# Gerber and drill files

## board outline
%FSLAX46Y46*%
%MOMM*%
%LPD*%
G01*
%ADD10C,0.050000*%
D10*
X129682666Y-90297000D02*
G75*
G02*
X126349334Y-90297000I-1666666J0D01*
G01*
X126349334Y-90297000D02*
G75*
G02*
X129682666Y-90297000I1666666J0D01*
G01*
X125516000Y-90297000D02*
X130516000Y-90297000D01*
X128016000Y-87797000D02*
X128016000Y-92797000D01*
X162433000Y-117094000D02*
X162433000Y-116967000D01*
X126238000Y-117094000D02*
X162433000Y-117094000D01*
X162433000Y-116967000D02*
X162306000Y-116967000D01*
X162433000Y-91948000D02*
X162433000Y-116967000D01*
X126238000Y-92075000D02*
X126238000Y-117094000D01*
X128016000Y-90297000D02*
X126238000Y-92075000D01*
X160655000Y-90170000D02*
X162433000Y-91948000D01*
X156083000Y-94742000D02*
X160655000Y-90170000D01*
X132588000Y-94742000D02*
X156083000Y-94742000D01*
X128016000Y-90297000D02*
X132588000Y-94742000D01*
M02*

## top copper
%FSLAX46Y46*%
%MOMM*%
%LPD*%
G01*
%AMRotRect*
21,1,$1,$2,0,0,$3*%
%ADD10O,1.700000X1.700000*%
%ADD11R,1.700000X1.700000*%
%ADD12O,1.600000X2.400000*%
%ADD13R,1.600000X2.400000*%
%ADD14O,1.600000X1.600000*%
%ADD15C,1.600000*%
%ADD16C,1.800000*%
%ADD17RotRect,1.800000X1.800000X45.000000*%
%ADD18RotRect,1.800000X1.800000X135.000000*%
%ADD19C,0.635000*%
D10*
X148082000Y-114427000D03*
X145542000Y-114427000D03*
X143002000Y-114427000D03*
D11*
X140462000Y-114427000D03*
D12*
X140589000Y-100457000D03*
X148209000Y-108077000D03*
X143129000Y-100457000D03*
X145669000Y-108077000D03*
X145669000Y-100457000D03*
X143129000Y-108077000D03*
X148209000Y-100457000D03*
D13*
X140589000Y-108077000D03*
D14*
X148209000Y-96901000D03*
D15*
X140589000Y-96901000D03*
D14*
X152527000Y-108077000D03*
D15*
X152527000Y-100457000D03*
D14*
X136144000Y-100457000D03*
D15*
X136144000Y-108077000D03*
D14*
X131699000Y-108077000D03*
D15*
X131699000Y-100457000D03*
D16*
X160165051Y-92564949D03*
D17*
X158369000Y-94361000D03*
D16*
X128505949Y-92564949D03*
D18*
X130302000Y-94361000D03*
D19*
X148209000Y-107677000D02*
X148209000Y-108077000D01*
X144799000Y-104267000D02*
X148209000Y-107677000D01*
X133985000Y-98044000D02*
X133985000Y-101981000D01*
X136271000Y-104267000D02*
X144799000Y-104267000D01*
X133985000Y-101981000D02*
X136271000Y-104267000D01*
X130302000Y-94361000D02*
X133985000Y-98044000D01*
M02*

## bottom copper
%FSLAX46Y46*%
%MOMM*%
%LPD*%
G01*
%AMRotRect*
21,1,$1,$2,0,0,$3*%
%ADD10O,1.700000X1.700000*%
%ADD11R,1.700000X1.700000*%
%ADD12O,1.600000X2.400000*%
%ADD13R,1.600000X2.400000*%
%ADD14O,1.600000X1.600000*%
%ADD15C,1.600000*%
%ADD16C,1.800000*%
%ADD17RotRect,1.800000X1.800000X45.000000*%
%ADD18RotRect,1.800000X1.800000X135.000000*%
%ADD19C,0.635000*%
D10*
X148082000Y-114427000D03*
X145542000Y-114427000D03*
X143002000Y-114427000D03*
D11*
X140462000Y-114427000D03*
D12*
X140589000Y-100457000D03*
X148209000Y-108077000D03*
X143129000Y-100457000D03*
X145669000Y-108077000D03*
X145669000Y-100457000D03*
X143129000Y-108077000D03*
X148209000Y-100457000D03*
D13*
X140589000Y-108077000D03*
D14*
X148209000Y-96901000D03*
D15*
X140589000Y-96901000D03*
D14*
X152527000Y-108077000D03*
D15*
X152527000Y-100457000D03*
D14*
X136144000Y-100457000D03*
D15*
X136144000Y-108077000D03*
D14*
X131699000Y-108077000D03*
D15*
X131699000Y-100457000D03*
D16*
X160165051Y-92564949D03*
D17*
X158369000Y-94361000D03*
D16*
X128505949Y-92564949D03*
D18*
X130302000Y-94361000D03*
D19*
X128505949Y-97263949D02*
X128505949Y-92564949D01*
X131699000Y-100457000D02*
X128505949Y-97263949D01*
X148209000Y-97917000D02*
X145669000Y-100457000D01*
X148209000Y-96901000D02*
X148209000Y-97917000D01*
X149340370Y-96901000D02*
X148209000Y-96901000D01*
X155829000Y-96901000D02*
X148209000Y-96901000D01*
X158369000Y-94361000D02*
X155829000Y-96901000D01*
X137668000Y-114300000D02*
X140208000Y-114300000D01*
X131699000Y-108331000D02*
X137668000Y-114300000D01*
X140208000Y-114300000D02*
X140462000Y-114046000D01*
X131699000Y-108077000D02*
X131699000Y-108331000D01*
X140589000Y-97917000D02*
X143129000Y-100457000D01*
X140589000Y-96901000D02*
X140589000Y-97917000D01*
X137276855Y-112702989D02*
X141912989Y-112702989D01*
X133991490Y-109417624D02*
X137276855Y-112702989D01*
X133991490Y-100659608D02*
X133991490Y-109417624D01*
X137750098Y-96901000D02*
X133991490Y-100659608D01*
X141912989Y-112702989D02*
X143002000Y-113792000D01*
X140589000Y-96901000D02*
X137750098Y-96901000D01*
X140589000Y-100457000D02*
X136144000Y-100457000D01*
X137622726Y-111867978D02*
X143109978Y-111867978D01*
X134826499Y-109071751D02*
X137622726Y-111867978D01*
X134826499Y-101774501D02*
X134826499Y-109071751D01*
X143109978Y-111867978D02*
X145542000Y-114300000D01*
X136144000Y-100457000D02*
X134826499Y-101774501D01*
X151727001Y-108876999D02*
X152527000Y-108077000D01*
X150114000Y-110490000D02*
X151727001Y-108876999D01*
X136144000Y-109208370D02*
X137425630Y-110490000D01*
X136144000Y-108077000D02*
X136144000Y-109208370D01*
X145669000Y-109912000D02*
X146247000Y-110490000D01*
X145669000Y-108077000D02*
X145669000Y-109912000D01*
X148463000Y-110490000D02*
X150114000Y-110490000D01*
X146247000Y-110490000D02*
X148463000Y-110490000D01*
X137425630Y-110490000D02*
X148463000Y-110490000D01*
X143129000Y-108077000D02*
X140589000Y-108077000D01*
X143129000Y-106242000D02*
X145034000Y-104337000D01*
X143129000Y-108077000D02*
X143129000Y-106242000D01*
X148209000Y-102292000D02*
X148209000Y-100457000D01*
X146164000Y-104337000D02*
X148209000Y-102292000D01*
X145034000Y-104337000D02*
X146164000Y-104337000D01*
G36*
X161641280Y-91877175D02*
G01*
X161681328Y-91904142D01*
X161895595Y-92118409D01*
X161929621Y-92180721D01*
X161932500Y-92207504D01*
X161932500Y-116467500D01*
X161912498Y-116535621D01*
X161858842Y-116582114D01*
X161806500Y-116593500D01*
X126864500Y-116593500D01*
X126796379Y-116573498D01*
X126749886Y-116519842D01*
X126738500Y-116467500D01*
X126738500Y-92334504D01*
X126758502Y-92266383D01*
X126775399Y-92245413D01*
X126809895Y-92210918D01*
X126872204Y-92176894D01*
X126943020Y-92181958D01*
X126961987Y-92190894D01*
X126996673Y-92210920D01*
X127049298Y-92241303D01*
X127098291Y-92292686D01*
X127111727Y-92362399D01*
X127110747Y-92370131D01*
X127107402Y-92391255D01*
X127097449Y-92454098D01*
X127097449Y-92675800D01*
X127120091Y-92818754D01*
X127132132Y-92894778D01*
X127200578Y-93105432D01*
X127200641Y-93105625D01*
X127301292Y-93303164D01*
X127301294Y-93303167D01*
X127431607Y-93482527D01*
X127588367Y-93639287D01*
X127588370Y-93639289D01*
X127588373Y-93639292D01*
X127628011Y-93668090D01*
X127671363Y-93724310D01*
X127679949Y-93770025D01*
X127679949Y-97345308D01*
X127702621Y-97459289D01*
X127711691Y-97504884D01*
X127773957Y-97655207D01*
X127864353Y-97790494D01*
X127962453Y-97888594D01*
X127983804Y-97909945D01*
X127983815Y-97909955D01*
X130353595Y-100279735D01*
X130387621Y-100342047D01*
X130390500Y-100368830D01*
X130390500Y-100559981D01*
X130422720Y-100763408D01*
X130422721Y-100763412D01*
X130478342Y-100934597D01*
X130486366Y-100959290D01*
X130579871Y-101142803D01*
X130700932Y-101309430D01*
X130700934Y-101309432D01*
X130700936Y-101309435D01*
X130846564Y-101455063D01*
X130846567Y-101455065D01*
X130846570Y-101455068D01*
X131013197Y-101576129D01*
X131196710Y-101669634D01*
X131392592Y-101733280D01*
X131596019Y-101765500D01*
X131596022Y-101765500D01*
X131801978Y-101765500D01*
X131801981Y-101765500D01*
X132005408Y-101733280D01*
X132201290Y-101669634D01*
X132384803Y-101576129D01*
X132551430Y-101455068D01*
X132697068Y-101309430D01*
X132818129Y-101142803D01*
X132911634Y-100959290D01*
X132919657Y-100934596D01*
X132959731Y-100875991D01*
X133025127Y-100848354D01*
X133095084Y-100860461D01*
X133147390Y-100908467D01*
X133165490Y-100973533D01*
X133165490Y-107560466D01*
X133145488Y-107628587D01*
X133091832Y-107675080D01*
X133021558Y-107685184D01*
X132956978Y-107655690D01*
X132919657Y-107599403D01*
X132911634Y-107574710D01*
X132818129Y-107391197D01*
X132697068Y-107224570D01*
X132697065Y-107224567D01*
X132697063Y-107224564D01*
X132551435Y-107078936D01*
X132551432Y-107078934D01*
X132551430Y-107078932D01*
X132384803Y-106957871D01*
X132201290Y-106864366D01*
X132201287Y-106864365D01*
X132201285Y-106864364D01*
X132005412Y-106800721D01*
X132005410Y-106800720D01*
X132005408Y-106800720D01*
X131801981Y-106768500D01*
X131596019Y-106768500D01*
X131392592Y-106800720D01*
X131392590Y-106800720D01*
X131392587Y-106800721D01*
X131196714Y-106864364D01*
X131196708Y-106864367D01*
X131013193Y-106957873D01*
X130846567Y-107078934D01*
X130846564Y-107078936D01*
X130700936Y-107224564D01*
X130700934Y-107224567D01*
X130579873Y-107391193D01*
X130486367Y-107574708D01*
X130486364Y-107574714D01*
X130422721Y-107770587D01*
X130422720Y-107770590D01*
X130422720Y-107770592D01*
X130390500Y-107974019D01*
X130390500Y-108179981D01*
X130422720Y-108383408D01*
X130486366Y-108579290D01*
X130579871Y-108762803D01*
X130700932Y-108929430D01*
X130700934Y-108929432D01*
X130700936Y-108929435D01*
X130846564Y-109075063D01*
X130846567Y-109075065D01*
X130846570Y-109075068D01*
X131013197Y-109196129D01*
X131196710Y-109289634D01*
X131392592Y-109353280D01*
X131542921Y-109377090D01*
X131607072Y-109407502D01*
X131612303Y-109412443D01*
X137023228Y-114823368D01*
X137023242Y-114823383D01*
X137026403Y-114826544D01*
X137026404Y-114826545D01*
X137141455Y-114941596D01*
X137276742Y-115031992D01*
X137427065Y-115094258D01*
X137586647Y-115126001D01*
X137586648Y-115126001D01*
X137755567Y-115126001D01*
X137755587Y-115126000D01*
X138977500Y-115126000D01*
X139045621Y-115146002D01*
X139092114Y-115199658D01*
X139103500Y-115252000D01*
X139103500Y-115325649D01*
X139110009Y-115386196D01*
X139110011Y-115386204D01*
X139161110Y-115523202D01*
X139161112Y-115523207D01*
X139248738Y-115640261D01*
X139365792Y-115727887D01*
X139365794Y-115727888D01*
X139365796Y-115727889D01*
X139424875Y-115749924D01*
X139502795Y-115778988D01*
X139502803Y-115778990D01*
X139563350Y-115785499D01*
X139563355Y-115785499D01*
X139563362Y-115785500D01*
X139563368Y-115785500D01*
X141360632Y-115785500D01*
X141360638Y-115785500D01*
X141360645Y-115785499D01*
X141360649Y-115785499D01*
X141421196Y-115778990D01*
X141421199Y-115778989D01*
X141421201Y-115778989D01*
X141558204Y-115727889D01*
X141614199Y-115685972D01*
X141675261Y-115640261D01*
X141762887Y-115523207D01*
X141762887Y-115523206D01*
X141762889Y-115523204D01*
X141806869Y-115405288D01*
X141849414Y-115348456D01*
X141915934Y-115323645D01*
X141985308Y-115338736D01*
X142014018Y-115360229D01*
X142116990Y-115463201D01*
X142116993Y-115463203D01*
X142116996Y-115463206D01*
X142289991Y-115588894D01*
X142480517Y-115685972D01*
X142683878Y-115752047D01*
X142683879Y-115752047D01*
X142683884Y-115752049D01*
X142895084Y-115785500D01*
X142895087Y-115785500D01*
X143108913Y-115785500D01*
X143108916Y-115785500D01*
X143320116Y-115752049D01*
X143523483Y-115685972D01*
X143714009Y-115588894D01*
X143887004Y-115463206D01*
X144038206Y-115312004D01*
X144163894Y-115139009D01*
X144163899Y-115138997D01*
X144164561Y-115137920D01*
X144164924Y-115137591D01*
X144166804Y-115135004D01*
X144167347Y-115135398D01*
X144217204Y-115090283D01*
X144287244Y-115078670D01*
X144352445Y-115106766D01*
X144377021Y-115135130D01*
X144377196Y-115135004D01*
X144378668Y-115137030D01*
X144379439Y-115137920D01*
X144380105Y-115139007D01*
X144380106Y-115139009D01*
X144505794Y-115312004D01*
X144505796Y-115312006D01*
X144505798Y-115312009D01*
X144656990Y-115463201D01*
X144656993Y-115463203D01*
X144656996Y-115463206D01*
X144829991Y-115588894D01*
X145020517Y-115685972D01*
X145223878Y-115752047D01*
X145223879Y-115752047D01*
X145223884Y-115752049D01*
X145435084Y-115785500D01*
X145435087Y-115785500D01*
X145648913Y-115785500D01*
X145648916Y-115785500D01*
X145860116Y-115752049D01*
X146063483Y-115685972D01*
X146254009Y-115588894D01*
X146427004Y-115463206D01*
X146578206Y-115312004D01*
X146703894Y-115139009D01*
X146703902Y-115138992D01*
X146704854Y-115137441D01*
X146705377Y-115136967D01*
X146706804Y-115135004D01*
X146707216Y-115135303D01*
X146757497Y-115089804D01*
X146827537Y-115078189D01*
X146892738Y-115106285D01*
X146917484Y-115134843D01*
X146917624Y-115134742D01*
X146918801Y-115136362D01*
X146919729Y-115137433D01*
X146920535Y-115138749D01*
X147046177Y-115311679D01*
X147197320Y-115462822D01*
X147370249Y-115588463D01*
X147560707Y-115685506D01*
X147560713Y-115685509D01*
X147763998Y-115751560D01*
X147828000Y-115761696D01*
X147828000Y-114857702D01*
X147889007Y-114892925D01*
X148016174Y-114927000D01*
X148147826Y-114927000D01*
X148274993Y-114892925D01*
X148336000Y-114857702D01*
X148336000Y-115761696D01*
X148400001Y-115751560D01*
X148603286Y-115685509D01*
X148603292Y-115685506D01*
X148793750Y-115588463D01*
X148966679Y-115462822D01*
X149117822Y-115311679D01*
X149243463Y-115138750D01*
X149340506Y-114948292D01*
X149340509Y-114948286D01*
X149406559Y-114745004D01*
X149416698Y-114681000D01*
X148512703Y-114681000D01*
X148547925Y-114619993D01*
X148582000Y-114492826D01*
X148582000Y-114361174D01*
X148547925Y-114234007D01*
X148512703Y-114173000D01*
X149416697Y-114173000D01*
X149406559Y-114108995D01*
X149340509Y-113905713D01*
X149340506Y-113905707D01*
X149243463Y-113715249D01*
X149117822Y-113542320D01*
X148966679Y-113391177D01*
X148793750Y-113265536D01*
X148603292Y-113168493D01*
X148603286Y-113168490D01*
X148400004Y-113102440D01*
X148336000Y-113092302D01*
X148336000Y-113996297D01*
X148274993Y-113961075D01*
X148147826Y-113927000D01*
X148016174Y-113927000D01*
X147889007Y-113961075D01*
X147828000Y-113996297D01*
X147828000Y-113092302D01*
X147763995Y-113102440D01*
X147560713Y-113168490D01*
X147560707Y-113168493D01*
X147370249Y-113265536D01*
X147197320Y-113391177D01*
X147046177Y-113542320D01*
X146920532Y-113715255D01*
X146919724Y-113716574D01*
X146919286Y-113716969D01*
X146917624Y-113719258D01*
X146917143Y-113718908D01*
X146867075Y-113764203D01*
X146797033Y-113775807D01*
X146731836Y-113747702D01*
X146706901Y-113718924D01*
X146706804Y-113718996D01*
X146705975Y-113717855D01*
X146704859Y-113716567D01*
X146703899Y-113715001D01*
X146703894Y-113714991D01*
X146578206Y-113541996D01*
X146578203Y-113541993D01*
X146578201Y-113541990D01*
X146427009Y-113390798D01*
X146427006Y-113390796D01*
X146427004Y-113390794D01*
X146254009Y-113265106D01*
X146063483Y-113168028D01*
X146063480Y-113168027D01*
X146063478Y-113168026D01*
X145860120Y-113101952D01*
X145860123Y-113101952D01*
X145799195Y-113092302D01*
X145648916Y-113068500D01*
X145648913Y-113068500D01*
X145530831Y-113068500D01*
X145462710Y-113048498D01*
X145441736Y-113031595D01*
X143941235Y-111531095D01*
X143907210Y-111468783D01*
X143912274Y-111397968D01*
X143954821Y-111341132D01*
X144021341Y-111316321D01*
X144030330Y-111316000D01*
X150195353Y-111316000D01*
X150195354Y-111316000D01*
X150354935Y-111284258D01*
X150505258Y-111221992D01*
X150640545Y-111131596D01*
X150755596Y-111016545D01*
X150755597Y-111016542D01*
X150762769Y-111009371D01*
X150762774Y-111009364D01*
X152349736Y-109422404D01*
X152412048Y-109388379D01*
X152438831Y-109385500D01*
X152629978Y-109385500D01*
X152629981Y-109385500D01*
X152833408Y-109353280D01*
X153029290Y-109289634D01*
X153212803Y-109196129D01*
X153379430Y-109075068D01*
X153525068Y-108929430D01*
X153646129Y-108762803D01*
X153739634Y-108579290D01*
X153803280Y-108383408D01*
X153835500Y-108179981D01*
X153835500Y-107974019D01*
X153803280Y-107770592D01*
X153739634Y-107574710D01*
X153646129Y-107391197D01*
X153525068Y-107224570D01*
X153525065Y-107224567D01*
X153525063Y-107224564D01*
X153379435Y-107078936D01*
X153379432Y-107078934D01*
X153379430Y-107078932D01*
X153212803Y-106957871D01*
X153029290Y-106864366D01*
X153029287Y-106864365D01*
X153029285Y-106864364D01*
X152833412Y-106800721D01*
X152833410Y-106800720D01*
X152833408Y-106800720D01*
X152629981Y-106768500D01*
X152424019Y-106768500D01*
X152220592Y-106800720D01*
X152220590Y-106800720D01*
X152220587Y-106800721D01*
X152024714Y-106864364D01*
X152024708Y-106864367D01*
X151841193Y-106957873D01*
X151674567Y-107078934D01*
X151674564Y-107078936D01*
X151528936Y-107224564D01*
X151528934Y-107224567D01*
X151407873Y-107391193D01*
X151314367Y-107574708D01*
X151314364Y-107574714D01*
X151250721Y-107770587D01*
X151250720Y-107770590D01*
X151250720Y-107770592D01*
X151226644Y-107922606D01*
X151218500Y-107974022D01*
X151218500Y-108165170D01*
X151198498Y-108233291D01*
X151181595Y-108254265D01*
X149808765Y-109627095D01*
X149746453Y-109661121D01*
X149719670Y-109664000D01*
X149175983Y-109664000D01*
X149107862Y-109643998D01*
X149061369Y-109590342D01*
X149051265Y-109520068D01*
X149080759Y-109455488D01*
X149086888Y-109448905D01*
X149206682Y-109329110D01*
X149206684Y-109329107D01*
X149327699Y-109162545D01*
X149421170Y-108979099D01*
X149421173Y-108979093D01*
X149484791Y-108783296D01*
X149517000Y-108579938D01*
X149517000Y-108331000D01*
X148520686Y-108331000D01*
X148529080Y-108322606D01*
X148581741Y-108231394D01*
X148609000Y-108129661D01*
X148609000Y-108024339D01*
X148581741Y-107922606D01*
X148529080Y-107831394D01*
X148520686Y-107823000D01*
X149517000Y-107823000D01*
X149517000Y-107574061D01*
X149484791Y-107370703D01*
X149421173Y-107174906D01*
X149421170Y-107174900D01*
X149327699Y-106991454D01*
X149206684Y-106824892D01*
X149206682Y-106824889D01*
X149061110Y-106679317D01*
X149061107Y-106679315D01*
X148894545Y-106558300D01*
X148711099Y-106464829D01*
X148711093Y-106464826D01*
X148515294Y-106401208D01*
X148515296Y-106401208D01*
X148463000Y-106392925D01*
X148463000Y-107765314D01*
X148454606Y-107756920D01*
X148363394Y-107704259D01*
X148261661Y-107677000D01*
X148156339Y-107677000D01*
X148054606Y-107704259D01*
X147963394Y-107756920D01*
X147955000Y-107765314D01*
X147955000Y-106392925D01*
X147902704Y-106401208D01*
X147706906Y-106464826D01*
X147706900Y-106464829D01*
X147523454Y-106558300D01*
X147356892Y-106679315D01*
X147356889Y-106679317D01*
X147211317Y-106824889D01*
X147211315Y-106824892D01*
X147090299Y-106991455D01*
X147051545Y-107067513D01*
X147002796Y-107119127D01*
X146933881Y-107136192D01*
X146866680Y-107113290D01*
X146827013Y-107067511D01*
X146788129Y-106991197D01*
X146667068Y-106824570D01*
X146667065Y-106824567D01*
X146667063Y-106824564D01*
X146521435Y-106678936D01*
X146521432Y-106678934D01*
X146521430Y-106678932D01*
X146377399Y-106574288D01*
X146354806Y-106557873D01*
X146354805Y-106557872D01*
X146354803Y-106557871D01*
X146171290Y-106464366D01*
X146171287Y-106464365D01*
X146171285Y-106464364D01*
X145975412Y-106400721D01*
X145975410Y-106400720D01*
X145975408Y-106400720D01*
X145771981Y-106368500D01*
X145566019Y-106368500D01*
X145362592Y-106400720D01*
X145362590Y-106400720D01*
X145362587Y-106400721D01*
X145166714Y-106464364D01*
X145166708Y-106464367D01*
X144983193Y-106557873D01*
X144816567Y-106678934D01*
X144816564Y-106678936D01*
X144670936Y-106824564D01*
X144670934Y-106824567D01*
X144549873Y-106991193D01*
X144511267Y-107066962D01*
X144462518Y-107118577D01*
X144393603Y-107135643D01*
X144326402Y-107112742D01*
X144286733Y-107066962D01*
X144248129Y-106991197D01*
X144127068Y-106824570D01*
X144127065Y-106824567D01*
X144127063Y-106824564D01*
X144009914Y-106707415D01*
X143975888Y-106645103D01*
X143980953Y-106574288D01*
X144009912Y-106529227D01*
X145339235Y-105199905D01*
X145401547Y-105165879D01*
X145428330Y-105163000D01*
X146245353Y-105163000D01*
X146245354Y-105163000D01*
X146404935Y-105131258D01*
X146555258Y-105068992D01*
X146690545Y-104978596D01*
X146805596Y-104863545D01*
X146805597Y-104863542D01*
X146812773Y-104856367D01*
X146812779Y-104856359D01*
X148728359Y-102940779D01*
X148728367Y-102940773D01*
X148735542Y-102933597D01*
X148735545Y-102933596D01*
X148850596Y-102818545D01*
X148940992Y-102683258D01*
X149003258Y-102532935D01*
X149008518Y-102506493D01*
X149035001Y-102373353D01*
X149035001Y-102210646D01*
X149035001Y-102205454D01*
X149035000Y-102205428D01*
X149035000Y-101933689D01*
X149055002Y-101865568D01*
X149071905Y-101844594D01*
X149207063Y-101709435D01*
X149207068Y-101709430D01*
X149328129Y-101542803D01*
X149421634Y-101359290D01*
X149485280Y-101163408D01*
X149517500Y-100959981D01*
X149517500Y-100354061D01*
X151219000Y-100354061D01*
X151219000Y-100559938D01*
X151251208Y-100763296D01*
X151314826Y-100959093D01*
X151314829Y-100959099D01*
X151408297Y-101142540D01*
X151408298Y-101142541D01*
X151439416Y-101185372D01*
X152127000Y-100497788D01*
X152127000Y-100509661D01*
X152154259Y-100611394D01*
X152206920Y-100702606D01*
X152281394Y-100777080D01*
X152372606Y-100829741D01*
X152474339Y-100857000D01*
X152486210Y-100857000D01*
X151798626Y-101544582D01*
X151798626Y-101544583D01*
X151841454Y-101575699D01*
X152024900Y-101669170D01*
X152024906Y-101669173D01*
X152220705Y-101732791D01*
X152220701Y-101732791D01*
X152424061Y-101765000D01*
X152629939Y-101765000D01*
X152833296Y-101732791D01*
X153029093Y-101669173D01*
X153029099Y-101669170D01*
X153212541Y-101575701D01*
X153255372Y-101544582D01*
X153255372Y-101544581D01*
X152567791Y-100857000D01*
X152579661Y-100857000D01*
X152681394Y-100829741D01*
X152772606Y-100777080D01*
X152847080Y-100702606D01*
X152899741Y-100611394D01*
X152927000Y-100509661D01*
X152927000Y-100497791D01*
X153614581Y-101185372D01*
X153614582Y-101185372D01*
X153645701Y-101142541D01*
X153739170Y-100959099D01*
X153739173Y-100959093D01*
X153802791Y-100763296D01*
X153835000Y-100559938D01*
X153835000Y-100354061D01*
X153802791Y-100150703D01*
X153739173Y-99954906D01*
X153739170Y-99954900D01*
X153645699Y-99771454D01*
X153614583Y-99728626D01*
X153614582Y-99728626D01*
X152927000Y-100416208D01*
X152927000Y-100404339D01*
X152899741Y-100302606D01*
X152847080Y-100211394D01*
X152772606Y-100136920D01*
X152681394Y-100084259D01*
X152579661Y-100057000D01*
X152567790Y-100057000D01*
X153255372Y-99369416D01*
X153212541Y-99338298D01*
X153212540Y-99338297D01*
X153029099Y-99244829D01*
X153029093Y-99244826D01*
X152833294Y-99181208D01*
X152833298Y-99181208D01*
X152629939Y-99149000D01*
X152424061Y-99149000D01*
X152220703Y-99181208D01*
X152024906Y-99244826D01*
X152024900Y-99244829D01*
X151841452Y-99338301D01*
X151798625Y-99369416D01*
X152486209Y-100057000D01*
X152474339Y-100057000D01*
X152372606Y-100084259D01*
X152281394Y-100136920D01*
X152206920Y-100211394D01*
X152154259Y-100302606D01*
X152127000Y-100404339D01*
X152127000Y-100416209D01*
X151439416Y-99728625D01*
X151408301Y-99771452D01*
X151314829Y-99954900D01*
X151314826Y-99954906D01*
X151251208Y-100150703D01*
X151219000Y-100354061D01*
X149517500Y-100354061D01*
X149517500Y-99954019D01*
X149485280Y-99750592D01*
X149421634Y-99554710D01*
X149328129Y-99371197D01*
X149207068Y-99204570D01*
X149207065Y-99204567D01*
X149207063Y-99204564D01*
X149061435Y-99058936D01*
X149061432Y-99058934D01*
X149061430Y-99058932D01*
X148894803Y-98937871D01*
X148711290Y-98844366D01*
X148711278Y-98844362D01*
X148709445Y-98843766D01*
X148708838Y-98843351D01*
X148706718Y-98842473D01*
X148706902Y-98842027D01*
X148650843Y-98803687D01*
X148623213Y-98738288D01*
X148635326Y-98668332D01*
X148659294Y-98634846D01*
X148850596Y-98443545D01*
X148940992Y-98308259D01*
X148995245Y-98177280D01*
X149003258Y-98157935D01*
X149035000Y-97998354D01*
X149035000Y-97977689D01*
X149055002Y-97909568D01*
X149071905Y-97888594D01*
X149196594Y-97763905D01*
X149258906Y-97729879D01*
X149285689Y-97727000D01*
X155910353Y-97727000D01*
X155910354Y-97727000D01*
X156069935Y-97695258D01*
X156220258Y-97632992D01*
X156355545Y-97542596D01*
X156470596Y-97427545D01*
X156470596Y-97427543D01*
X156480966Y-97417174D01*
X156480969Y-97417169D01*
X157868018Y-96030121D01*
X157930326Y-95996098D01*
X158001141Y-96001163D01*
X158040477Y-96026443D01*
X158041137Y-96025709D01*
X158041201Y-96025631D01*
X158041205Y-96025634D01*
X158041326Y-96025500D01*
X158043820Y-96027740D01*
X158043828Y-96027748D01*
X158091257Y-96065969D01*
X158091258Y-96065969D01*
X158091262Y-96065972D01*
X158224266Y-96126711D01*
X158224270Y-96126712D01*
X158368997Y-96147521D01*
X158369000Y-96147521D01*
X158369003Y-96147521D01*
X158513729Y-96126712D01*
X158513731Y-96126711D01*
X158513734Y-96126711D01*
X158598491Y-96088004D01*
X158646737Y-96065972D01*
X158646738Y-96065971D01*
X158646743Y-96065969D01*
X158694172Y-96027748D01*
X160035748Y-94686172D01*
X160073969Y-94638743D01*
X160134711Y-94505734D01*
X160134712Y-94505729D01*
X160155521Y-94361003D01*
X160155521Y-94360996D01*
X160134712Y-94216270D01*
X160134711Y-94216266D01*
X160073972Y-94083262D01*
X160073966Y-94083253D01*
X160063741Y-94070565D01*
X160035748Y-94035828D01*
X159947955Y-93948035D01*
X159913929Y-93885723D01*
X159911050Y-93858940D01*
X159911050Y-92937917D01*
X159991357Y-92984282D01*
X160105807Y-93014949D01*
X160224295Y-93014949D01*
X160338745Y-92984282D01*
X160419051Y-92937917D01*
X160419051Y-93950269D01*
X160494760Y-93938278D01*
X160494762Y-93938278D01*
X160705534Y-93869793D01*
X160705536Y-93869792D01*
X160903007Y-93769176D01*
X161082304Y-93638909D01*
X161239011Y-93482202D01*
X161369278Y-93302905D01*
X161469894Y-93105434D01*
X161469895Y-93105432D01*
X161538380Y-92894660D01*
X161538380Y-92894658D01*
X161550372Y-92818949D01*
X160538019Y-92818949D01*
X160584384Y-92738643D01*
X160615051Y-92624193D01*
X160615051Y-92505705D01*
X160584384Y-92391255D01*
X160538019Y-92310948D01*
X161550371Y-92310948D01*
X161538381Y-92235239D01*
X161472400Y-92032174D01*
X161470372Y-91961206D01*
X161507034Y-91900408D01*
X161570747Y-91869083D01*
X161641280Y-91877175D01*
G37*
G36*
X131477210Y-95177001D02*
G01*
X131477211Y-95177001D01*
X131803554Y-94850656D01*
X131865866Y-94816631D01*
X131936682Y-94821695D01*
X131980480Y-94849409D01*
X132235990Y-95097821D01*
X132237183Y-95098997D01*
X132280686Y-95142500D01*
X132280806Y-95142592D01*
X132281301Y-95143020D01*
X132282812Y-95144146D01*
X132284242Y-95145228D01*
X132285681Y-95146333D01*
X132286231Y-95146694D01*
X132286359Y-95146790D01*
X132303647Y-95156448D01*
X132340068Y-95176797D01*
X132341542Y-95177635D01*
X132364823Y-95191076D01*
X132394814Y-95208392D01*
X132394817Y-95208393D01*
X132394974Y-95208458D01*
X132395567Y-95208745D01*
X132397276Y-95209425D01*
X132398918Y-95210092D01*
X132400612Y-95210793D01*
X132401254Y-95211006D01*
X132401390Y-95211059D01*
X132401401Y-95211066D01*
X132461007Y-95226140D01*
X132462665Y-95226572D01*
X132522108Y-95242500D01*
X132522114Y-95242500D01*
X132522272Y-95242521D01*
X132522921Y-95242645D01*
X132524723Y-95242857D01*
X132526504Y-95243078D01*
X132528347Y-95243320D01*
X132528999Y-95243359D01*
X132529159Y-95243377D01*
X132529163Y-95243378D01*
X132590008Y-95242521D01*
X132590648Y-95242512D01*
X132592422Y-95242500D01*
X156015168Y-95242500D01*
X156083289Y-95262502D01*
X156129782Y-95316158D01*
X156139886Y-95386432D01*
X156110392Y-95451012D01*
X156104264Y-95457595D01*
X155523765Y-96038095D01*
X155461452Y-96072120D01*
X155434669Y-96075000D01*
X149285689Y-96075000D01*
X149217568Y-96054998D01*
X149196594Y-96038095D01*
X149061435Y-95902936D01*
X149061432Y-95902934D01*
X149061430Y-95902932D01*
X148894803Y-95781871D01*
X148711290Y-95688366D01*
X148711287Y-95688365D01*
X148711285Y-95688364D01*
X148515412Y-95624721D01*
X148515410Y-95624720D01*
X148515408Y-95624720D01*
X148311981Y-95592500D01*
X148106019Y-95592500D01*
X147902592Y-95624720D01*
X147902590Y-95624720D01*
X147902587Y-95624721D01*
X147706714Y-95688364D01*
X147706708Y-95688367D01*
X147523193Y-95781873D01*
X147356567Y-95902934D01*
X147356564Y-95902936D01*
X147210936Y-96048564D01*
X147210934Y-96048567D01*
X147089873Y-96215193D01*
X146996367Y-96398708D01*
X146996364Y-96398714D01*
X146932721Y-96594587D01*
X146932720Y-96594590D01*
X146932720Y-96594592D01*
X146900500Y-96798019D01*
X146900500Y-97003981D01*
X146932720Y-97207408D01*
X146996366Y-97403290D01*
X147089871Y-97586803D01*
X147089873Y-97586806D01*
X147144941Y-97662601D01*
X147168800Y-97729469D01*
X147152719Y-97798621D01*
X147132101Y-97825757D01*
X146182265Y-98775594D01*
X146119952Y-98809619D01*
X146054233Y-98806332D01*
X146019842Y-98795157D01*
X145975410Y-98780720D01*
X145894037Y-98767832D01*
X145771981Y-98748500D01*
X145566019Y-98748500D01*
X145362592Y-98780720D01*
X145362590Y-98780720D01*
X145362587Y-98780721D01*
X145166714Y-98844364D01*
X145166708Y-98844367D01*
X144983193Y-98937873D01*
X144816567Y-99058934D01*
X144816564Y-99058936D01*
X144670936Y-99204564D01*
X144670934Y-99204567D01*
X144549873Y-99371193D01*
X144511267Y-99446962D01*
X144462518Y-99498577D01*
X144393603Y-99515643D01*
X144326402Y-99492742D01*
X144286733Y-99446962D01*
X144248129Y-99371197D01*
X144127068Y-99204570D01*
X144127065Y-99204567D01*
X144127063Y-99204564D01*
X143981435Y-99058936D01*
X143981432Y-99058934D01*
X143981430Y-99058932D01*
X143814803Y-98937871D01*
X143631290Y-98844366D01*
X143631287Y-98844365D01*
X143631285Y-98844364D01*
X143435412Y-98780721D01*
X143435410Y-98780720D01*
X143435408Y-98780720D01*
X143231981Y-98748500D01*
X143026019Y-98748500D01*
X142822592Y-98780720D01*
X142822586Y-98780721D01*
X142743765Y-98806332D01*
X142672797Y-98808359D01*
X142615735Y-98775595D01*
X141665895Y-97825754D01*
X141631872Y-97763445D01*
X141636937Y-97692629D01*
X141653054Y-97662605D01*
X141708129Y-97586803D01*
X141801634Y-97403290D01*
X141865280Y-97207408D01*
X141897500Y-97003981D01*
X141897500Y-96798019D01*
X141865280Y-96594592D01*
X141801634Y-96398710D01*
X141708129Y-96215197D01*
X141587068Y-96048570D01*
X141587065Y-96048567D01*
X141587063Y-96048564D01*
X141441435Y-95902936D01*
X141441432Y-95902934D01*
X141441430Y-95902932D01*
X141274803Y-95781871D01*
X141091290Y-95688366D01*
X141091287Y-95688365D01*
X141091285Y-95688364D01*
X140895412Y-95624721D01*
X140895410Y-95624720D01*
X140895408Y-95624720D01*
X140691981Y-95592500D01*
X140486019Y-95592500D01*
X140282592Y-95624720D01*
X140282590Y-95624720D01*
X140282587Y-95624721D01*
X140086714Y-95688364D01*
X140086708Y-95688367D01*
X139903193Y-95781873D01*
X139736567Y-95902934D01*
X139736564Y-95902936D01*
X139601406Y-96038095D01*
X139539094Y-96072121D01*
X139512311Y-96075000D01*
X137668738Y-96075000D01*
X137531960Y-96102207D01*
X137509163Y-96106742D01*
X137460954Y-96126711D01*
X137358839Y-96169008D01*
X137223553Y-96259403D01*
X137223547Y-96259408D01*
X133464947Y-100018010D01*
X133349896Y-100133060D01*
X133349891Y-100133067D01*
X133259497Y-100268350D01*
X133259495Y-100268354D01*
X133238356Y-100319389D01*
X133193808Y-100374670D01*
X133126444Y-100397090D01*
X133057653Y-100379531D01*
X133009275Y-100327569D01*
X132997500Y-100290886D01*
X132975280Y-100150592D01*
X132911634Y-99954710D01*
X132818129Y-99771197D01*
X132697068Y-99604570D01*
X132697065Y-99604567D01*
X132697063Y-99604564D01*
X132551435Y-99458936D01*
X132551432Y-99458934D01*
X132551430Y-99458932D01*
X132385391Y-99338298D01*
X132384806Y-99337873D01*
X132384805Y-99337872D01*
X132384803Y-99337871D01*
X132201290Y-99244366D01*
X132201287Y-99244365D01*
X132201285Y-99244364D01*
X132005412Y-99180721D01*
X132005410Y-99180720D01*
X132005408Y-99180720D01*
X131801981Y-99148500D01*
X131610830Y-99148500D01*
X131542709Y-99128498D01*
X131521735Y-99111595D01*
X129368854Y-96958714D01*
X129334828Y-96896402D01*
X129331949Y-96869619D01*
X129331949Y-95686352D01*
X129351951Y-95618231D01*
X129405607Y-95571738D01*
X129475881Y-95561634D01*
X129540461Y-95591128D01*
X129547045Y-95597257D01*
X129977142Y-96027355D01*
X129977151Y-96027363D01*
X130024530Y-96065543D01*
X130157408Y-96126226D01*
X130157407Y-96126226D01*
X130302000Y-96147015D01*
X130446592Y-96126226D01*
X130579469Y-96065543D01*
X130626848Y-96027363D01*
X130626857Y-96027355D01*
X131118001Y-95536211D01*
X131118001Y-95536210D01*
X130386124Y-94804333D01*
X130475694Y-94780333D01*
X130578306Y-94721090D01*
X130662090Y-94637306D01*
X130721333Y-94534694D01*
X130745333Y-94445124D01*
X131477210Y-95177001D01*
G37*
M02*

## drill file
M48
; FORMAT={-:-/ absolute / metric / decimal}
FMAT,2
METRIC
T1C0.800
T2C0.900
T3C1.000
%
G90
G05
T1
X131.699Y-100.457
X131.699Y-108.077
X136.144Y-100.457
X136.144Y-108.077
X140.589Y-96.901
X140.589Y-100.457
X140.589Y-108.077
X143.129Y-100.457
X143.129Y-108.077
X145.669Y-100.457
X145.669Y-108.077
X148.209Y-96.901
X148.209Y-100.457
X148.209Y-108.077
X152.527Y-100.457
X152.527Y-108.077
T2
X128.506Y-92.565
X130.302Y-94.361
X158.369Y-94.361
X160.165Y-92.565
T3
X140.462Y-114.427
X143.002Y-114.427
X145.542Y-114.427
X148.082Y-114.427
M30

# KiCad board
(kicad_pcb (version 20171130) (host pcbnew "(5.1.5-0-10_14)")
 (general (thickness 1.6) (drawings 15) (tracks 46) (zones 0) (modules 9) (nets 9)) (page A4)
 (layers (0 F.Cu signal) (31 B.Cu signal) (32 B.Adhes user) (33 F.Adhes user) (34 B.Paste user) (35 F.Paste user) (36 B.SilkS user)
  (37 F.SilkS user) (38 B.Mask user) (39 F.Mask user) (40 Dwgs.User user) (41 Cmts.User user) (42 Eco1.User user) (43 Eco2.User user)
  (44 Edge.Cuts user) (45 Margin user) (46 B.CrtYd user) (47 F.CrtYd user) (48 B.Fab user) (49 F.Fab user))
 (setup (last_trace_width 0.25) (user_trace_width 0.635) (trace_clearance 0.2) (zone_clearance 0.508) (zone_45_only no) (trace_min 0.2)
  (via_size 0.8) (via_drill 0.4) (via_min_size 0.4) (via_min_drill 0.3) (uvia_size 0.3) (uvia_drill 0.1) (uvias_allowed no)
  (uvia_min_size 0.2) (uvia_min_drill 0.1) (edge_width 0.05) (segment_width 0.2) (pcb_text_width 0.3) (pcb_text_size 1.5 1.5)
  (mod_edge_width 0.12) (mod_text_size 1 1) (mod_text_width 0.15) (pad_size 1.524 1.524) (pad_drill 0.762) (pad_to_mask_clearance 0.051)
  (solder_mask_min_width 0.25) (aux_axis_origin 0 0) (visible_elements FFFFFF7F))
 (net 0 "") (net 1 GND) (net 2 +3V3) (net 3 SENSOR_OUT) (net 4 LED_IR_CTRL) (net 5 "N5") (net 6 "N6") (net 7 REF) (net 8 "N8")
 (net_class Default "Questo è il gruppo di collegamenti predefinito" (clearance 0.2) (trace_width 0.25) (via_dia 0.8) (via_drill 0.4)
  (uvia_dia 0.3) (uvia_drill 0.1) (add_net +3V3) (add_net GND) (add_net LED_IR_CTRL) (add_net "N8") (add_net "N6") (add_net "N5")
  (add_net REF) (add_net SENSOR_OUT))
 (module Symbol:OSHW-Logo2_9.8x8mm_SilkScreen (layer F.Cu) (at 156.718 111.76)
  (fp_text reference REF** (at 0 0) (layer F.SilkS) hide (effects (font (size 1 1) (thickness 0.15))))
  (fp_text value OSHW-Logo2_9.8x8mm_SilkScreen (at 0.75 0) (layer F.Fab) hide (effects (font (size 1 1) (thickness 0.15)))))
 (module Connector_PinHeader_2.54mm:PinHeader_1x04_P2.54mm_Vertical (layer F.Cu) (at 140.462 114.427 90)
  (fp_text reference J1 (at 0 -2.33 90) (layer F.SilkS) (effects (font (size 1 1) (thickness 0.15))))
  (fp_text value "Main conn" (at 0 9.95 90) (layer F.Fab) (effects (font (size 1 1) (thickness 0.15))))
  (pad 4 thru_hole oval (at 0 7.62 90) (size 1.7 1.7) (drill 1) (layers *.Cu *.Mask) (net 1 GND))
  (pad 3 thru_hole oval (at 0 5.08 90) (size 1.7 1.7) (drill 1) (layers *.Cu *.Mask) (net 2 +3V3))
  (pad 2 thru_hole oval (at 0 2.54 90) (size 1.7 1.7) (drill 1) (layers *.Cu *.Mask) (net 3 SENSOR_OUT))
  (pad 1 thru_hole rect (at 0 0 90) (size 1.7 1.7) (drill 1) (layers *.Cu *.Mask) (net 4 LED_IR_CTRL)))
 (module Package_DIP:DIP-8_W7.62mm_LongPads (layer F.Cu) (at 140.589 108.077 90)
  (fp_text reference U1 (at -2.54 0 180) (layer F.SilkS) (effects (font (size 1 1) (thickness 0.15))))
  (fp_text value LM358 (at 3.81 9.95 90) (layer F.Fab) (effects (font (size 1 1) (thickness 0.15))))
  (pad 8 thru_hole oval (at 7.62 0 90) (size 2.4 1.6) (drill 0.8) (layers *.Cu *.Mask) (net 2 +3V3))
  (pad 4 thru_hole oval (at 0 7.62 90) (size 2.4 1.6) (drill 0.8) (layers *.Cu *.Mask) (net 1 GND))
  (pad 7 thru_hole oval (at 7.62 2.54 90) (size 2.4 1.6) (drill 0.8) (layers *.Cu *.Mask) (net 3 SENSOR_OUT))
  (pad 3 thru_hole oval (at 0 5.08 90) (size 2.4 1.6) (drill 0.8) (layers *.Cu *.Mask) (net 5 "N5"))
  (pad 6 thru_hole oval (at 7.62 5.08 90) (size 2.4 1.6) (drill 0.8) (layers *.Cu *.Mask) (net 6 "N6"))
  (pad 2 thru_hole oval (at 0 2.54 90) (size 2.4 1.6) (drill 0.8) (layers *.Cu *.Mask) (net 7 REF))
  (pad 5 thru_hole oval (at 7.62 7.62 90) (size 2.4 1.6) (drill 0.8) (layers *.Cu *.Mask) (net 7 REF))
  (pad 1 thru_hole rect (at 0 0 90) (size 2.4 1.6) (drill 0.8) (layers *.Cu *.Mask) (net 7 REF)))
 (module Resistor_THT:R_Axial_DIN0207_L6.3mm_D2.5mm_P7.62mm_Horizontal (layer F.Cu) (at 140.589 96.901)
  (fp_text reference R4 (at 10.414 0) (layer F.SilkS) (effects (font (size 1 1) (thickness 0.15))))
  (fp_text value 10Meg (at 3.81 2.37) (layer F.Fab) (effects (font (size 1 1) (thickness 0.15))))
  (pad 2 thru_hole oval (at 7.62 0) (size 1.6 1.6) (drill 0.8) (layers *.Cu *.Mask) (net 6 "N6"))
  (pad 1 thru_hole circle (at 0 0) (size 1.6 1.6) (drill 0.8) (layers *.Cu *.Mask) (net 3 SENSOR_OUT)))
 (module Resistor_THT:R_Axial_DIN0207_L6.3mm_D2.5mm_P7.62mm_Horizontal (layer F.Cu) (at 152.527 100.457 270)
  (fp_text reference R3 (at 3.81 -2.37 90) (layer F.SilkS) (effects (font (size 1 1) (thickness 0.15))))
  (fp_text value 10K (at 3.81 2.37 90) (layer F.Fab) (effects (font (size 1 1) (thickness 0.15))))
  (pad 2 thru_hole oval (at 7.62 0 270) (size 1.6 1.6) (drill 0.8) (layers *.Cu *.Mask) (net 5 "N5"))
  (pad 1 thru_hole circle (at 0 0 270) (size 1.6 1.6) (drill 0.8) (layers *.Cu *.Mask) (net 1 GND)))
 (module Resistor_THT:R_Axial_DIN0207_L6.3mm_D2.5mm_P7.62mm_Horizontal (layer F.Cu) (at 136.144 108.077 90)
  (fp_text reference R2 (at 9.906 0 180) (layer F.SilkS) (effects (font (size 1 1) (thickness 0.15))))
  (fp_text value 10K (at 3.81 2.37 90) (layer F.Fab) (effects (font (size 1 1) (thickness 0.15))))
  (pad 2 thru_hole oval (at 7.62 0 90) (size 1.6 1.6) (drill 0.8) (layers *.Cu *.Mask) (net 2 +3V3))
  (pad 1 thru_hole circle (at 0 0 90) (size 1.6 1.6) (drill 0.8) (layers *.Cu *.Mask) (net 5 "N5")))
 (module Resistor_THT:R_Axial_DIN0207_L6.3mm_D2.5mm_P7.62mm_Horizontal (layer F.Cu) (at 131.699 100.457 270)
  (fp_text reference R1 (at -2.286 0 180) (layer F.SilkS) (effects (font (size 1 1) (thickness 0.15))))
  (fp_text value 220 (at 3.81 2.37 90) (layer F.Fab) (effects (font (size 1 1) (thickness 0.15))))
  (pad 2 thru_hole oval (at 7.62 0 270) (size 1.6 1.6) (drill 0.8) (layers *.Cu *.Mask) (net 4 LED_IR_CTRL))
  (pad 1 thru_hole circle (at 0 0 270) (size 1.6 1.6) (drill 0.8) (layers *.Cu *.Mask) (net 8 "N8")))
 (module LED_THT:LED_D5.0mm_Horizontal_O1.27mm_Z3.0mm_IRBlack (layer B.Cu) (at 158.369 94.361 45)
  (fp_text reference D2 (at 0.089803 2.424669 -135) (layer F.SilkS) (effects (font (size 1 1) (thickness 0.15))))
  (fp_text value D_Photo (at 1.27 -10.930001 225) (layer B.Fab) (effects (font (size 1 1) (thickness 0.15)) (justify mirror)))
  (pad 2 thru_hole circle (at 2.54 0 45) (size 1.8 1.8) (drill 0.9) (layers *.Cu *.Mask) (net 1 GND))
  (pad 1 thru_hole rect (at 0 0 45) (size 1.8 1.8) (drill 0.9) (layers *.Cu *.Mask) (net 6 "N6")))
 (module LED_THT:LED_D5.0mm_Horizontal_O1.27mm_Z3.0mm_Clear (layer F.Cu) (at 130.302 94.361 135)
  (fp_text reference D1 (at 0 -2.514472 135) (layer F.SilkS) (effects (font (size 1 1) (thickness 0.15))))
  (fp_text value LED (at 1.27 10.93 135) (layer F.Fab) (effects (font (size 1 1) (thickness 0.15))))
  (pad 2 thru_hole circle (at 2.54 0 135) (size 1.8 1.8) (drill 0.9) (layers *.Cu *.Mask) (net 8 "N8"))
  (pad 1 thru_hole rect (at 0 0 135) (size 1.8 1.8) (drill 0.9) (layers *.Cu *.Mask) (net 1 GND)))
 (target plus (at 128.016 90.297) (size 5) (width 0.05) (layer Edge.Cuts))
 (gr_line (start 162.433 117.094) (end 162.433 116.967) (layer Edge.Cuts) (width 0.05))
 (gr_line (start 126.238 117.094) (end 162.433 117.094) (layer Edge.Cuts) (width 0.05))
 (gr_line (start 162.433 116.967) (end 162.306 116.967) (layer Edge.Cuts) (width 0.05))
 (gr_line (start 162.433 91.948) (end 162.433 116.967) (layer Edge.Cuts) (width 0.05))
 (gr_line (start 126.238 92.075) (end 126.238 117.094) (layer Edge.Cuts) (width 0.05))
 (gr_line (start 128.016 90.297) (end 126.238 92.075) (layer Edge.Cuts) (width 0.05))
 (gr_line (start 160.655 90.17) (end 162.433 91.948) (layer Edge.Cuts) (width 0.05))
 (gr_line (start 156.083 94.742) (end 160.655 90.17) (layer Edge.Cuts) (width 0.05))
 (gr_line (start 132.588 94.742) (end 156.083 94.742) (layer Edge.Cuts) (width 0.05))
 (gr_line (start 128.016 90.297) (end 132.588 94.742) (layer Edge.Cuts) (width 0.05))
 (segment (start 128.505949 97.263949) (end 128.505949 92.564949) (width 0.635) (layer B.Cu) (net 8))
 (segment (start 131.699 100.457) (end 128.505949 97.263949) (width 0.635) (layer B.Cu) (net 8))
 (segment (start 148.209 107.677) (end 148.209 108.077) (width 0.635) (layer F.Cu) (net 1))
 (segment (start 144.799 104.267) (end 148.209 107.677) (width 0.635) (layer F.Cu) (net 1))
 (segment (start 133.985 98.044) (end 133.985 101.981) (width 0.635) (layer F.Cu) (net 1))
 (segment (start 136.271 104.267) (end 144.799 104.267) (width 0.635) (layer F.Cu) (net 1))
 (segment (start 133.985 101.981) (end 136.271 104.267) (width 0.635) (layer F.Cu) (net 1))
 (segment (start 130.302 94.361) (end 133.985 98.044) (width 0.635) (layer F.Cu) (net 1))
 (segment (start 148.209 97.917) (end 145.669 100.457) (width 0.635) (layer B.Cu) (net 6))
 (segment (start 148.209 96.901) (end 148.209 97.917) (width 0.635) (layer B.Cu) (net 6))
 (segment (start 149.34037 96.901) (end 148.209 96.901) (width 0.635) (layer B.Cu) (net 6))
 (segment (start 155.829 96.901) (end 148.209 96.901) (width 0.635) (layer B.Cu) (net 6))
 (segment (start 158.369 94.361) (end 155.829 96.901) (width 0.635) (layer B.Cu) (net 6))
 (segment (start 137.668 114.3) (end 140.208 114.3) (width 0.635) (layer B.Cu) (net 4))
 (segment (start 131.699 108.331) (end 137.668 114.3) (width 0.635) (layer B.Cu) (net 4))
 (segment (start 140.208 114.3) (end 140.462 114.046) (width 0.635) (layer B.Cu) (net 4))
 (segment (start 131.699 108.077) (end 131.699 108.331) (width 0.635) (layer B.Cu) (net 4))
 (segment (start 140.589 97.917) (end 143.129 100.457) (width 0.635) (layer B.Cu) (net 3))
 (segment (start 140.589 96.901) (end 140.589 97.917) (width 0.635) (layer B.Cu) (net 3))
 (segment (start 137.276855 112.702989) (end 141.912989 112.702989) (width 0.635) (layer B.Cu) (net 3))
 (segment (start 133.99149 109.417624) (end 137.276855 112.702989) (width 0.635) (layer B.Cu) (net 3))
 (segment (start 133.99149 100.659608) (end 133.99149 109.417624) (width 0.635) (layer B.Cu) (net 3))
 (segment (start 137.750098 96.901) (end 133.99149 100.659608) (width 0.635) (layer B.Cu) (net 3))
 (segment (start 141.912989 112.702989) (end 143.002 113.792) (width 0.635) (layer B.Cu) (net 3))
 (segment (start 140.589 96.901) (end 137.750098 96.901) (width 0.635) (layer B.Cu) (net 3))
 (segment (start 140.589 100.457) (end 136.144 100.457) (width 0.635) (layer B.Cu) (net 2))
 (segment (start 137.622726 111.867978) (end 143.109978 111.867978) (width 0.635) (layer B.Cu) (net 2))
 (segment (start 134.826499 109.071751) (end 137.622726 111.867978) (width 0.635) (layer B.Cu) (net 2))
 (segment (start 134.826499 101.774501) (end 134.826499 109.071751) (width 0.635) (layer B.Cu) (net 2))
 (segment (start 143.109978 111.867978) (end 145.542 114.3) (width 0.635) (layer B.Cu) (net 2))
 (segment (start 136.144 100.457) (end 134.826499 101.774501) (width 0.635) (layer B.Cu) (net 2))
 (segment (start 151.727001 108.876999) (end 152.527 108.077) (width 0.635) (layer B.Cu) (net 5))
 (segment (start 150.114 110.49) (end 151.727001 108.876999) (width 0.635) (layer B.Cu) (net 5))
 (segment (start 136.144 109.20837) (end 137.42563 110.49) (width 0.635) (layer B.Cu) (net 5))
 (segment (start 136.144 108.077) (end 136.144 109.20837) (width 0.635) (layer B.Cu) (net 5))
 (segment (start 145.669 109.912) (end 146.247 110.49) (width 0.635) (layer B.Cu) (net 5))
 (segment (start 145.669 108.077) (end 145.669 109.912) (width 0.635) (layer B.Cu) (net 5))
 (segment (start 148.463 110.49) (end 150.114 110.49) (width 0.635) (layer B.Cu) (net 5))
 (segment (start 146.247 110.49) (end 148.463 110.49) (width 0.635) (layer B.Cu) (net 5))
 (segment (start 137.42563 110.49) (end 148.463 110.49) (width 0.635) (layer B.Cu) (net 5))
 (segment (start 143.129 108.077) (end 140.589 108.077) (width 0.635) (layer B.Cu) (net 7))
 (segment (start 143.129 106.242) (end 145.034 104.337) (width 0.635) (layer B.Cu) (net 7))
 (segment (start 143.129 108.077) (end 143.129 106.242) (width 0.635) (layer B.Cu) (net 7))
 (segment (start 148.209 102.292) (end 148.209 100.457) (width 0.635) (layer B.Cu) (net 7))
 (segment (start 146.164 104.337) (end 148.209 102.292) (width 0.635) (layer B.Cu) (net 7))
 (segment (start 145.034 104.337) (end 146.164 104.337) (width 0.635) (layer B.Cu) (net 7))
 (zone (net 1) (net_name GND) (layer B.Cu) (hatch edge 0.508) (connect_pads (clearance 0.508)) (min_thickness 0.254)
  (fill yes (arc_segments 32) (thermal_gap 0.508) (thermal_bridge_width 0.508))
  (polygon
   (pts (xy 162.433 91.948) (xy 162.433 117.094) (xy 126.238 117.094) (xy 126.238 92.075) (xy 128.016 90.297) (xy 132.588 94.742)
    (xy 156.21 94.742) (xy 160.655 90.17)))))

